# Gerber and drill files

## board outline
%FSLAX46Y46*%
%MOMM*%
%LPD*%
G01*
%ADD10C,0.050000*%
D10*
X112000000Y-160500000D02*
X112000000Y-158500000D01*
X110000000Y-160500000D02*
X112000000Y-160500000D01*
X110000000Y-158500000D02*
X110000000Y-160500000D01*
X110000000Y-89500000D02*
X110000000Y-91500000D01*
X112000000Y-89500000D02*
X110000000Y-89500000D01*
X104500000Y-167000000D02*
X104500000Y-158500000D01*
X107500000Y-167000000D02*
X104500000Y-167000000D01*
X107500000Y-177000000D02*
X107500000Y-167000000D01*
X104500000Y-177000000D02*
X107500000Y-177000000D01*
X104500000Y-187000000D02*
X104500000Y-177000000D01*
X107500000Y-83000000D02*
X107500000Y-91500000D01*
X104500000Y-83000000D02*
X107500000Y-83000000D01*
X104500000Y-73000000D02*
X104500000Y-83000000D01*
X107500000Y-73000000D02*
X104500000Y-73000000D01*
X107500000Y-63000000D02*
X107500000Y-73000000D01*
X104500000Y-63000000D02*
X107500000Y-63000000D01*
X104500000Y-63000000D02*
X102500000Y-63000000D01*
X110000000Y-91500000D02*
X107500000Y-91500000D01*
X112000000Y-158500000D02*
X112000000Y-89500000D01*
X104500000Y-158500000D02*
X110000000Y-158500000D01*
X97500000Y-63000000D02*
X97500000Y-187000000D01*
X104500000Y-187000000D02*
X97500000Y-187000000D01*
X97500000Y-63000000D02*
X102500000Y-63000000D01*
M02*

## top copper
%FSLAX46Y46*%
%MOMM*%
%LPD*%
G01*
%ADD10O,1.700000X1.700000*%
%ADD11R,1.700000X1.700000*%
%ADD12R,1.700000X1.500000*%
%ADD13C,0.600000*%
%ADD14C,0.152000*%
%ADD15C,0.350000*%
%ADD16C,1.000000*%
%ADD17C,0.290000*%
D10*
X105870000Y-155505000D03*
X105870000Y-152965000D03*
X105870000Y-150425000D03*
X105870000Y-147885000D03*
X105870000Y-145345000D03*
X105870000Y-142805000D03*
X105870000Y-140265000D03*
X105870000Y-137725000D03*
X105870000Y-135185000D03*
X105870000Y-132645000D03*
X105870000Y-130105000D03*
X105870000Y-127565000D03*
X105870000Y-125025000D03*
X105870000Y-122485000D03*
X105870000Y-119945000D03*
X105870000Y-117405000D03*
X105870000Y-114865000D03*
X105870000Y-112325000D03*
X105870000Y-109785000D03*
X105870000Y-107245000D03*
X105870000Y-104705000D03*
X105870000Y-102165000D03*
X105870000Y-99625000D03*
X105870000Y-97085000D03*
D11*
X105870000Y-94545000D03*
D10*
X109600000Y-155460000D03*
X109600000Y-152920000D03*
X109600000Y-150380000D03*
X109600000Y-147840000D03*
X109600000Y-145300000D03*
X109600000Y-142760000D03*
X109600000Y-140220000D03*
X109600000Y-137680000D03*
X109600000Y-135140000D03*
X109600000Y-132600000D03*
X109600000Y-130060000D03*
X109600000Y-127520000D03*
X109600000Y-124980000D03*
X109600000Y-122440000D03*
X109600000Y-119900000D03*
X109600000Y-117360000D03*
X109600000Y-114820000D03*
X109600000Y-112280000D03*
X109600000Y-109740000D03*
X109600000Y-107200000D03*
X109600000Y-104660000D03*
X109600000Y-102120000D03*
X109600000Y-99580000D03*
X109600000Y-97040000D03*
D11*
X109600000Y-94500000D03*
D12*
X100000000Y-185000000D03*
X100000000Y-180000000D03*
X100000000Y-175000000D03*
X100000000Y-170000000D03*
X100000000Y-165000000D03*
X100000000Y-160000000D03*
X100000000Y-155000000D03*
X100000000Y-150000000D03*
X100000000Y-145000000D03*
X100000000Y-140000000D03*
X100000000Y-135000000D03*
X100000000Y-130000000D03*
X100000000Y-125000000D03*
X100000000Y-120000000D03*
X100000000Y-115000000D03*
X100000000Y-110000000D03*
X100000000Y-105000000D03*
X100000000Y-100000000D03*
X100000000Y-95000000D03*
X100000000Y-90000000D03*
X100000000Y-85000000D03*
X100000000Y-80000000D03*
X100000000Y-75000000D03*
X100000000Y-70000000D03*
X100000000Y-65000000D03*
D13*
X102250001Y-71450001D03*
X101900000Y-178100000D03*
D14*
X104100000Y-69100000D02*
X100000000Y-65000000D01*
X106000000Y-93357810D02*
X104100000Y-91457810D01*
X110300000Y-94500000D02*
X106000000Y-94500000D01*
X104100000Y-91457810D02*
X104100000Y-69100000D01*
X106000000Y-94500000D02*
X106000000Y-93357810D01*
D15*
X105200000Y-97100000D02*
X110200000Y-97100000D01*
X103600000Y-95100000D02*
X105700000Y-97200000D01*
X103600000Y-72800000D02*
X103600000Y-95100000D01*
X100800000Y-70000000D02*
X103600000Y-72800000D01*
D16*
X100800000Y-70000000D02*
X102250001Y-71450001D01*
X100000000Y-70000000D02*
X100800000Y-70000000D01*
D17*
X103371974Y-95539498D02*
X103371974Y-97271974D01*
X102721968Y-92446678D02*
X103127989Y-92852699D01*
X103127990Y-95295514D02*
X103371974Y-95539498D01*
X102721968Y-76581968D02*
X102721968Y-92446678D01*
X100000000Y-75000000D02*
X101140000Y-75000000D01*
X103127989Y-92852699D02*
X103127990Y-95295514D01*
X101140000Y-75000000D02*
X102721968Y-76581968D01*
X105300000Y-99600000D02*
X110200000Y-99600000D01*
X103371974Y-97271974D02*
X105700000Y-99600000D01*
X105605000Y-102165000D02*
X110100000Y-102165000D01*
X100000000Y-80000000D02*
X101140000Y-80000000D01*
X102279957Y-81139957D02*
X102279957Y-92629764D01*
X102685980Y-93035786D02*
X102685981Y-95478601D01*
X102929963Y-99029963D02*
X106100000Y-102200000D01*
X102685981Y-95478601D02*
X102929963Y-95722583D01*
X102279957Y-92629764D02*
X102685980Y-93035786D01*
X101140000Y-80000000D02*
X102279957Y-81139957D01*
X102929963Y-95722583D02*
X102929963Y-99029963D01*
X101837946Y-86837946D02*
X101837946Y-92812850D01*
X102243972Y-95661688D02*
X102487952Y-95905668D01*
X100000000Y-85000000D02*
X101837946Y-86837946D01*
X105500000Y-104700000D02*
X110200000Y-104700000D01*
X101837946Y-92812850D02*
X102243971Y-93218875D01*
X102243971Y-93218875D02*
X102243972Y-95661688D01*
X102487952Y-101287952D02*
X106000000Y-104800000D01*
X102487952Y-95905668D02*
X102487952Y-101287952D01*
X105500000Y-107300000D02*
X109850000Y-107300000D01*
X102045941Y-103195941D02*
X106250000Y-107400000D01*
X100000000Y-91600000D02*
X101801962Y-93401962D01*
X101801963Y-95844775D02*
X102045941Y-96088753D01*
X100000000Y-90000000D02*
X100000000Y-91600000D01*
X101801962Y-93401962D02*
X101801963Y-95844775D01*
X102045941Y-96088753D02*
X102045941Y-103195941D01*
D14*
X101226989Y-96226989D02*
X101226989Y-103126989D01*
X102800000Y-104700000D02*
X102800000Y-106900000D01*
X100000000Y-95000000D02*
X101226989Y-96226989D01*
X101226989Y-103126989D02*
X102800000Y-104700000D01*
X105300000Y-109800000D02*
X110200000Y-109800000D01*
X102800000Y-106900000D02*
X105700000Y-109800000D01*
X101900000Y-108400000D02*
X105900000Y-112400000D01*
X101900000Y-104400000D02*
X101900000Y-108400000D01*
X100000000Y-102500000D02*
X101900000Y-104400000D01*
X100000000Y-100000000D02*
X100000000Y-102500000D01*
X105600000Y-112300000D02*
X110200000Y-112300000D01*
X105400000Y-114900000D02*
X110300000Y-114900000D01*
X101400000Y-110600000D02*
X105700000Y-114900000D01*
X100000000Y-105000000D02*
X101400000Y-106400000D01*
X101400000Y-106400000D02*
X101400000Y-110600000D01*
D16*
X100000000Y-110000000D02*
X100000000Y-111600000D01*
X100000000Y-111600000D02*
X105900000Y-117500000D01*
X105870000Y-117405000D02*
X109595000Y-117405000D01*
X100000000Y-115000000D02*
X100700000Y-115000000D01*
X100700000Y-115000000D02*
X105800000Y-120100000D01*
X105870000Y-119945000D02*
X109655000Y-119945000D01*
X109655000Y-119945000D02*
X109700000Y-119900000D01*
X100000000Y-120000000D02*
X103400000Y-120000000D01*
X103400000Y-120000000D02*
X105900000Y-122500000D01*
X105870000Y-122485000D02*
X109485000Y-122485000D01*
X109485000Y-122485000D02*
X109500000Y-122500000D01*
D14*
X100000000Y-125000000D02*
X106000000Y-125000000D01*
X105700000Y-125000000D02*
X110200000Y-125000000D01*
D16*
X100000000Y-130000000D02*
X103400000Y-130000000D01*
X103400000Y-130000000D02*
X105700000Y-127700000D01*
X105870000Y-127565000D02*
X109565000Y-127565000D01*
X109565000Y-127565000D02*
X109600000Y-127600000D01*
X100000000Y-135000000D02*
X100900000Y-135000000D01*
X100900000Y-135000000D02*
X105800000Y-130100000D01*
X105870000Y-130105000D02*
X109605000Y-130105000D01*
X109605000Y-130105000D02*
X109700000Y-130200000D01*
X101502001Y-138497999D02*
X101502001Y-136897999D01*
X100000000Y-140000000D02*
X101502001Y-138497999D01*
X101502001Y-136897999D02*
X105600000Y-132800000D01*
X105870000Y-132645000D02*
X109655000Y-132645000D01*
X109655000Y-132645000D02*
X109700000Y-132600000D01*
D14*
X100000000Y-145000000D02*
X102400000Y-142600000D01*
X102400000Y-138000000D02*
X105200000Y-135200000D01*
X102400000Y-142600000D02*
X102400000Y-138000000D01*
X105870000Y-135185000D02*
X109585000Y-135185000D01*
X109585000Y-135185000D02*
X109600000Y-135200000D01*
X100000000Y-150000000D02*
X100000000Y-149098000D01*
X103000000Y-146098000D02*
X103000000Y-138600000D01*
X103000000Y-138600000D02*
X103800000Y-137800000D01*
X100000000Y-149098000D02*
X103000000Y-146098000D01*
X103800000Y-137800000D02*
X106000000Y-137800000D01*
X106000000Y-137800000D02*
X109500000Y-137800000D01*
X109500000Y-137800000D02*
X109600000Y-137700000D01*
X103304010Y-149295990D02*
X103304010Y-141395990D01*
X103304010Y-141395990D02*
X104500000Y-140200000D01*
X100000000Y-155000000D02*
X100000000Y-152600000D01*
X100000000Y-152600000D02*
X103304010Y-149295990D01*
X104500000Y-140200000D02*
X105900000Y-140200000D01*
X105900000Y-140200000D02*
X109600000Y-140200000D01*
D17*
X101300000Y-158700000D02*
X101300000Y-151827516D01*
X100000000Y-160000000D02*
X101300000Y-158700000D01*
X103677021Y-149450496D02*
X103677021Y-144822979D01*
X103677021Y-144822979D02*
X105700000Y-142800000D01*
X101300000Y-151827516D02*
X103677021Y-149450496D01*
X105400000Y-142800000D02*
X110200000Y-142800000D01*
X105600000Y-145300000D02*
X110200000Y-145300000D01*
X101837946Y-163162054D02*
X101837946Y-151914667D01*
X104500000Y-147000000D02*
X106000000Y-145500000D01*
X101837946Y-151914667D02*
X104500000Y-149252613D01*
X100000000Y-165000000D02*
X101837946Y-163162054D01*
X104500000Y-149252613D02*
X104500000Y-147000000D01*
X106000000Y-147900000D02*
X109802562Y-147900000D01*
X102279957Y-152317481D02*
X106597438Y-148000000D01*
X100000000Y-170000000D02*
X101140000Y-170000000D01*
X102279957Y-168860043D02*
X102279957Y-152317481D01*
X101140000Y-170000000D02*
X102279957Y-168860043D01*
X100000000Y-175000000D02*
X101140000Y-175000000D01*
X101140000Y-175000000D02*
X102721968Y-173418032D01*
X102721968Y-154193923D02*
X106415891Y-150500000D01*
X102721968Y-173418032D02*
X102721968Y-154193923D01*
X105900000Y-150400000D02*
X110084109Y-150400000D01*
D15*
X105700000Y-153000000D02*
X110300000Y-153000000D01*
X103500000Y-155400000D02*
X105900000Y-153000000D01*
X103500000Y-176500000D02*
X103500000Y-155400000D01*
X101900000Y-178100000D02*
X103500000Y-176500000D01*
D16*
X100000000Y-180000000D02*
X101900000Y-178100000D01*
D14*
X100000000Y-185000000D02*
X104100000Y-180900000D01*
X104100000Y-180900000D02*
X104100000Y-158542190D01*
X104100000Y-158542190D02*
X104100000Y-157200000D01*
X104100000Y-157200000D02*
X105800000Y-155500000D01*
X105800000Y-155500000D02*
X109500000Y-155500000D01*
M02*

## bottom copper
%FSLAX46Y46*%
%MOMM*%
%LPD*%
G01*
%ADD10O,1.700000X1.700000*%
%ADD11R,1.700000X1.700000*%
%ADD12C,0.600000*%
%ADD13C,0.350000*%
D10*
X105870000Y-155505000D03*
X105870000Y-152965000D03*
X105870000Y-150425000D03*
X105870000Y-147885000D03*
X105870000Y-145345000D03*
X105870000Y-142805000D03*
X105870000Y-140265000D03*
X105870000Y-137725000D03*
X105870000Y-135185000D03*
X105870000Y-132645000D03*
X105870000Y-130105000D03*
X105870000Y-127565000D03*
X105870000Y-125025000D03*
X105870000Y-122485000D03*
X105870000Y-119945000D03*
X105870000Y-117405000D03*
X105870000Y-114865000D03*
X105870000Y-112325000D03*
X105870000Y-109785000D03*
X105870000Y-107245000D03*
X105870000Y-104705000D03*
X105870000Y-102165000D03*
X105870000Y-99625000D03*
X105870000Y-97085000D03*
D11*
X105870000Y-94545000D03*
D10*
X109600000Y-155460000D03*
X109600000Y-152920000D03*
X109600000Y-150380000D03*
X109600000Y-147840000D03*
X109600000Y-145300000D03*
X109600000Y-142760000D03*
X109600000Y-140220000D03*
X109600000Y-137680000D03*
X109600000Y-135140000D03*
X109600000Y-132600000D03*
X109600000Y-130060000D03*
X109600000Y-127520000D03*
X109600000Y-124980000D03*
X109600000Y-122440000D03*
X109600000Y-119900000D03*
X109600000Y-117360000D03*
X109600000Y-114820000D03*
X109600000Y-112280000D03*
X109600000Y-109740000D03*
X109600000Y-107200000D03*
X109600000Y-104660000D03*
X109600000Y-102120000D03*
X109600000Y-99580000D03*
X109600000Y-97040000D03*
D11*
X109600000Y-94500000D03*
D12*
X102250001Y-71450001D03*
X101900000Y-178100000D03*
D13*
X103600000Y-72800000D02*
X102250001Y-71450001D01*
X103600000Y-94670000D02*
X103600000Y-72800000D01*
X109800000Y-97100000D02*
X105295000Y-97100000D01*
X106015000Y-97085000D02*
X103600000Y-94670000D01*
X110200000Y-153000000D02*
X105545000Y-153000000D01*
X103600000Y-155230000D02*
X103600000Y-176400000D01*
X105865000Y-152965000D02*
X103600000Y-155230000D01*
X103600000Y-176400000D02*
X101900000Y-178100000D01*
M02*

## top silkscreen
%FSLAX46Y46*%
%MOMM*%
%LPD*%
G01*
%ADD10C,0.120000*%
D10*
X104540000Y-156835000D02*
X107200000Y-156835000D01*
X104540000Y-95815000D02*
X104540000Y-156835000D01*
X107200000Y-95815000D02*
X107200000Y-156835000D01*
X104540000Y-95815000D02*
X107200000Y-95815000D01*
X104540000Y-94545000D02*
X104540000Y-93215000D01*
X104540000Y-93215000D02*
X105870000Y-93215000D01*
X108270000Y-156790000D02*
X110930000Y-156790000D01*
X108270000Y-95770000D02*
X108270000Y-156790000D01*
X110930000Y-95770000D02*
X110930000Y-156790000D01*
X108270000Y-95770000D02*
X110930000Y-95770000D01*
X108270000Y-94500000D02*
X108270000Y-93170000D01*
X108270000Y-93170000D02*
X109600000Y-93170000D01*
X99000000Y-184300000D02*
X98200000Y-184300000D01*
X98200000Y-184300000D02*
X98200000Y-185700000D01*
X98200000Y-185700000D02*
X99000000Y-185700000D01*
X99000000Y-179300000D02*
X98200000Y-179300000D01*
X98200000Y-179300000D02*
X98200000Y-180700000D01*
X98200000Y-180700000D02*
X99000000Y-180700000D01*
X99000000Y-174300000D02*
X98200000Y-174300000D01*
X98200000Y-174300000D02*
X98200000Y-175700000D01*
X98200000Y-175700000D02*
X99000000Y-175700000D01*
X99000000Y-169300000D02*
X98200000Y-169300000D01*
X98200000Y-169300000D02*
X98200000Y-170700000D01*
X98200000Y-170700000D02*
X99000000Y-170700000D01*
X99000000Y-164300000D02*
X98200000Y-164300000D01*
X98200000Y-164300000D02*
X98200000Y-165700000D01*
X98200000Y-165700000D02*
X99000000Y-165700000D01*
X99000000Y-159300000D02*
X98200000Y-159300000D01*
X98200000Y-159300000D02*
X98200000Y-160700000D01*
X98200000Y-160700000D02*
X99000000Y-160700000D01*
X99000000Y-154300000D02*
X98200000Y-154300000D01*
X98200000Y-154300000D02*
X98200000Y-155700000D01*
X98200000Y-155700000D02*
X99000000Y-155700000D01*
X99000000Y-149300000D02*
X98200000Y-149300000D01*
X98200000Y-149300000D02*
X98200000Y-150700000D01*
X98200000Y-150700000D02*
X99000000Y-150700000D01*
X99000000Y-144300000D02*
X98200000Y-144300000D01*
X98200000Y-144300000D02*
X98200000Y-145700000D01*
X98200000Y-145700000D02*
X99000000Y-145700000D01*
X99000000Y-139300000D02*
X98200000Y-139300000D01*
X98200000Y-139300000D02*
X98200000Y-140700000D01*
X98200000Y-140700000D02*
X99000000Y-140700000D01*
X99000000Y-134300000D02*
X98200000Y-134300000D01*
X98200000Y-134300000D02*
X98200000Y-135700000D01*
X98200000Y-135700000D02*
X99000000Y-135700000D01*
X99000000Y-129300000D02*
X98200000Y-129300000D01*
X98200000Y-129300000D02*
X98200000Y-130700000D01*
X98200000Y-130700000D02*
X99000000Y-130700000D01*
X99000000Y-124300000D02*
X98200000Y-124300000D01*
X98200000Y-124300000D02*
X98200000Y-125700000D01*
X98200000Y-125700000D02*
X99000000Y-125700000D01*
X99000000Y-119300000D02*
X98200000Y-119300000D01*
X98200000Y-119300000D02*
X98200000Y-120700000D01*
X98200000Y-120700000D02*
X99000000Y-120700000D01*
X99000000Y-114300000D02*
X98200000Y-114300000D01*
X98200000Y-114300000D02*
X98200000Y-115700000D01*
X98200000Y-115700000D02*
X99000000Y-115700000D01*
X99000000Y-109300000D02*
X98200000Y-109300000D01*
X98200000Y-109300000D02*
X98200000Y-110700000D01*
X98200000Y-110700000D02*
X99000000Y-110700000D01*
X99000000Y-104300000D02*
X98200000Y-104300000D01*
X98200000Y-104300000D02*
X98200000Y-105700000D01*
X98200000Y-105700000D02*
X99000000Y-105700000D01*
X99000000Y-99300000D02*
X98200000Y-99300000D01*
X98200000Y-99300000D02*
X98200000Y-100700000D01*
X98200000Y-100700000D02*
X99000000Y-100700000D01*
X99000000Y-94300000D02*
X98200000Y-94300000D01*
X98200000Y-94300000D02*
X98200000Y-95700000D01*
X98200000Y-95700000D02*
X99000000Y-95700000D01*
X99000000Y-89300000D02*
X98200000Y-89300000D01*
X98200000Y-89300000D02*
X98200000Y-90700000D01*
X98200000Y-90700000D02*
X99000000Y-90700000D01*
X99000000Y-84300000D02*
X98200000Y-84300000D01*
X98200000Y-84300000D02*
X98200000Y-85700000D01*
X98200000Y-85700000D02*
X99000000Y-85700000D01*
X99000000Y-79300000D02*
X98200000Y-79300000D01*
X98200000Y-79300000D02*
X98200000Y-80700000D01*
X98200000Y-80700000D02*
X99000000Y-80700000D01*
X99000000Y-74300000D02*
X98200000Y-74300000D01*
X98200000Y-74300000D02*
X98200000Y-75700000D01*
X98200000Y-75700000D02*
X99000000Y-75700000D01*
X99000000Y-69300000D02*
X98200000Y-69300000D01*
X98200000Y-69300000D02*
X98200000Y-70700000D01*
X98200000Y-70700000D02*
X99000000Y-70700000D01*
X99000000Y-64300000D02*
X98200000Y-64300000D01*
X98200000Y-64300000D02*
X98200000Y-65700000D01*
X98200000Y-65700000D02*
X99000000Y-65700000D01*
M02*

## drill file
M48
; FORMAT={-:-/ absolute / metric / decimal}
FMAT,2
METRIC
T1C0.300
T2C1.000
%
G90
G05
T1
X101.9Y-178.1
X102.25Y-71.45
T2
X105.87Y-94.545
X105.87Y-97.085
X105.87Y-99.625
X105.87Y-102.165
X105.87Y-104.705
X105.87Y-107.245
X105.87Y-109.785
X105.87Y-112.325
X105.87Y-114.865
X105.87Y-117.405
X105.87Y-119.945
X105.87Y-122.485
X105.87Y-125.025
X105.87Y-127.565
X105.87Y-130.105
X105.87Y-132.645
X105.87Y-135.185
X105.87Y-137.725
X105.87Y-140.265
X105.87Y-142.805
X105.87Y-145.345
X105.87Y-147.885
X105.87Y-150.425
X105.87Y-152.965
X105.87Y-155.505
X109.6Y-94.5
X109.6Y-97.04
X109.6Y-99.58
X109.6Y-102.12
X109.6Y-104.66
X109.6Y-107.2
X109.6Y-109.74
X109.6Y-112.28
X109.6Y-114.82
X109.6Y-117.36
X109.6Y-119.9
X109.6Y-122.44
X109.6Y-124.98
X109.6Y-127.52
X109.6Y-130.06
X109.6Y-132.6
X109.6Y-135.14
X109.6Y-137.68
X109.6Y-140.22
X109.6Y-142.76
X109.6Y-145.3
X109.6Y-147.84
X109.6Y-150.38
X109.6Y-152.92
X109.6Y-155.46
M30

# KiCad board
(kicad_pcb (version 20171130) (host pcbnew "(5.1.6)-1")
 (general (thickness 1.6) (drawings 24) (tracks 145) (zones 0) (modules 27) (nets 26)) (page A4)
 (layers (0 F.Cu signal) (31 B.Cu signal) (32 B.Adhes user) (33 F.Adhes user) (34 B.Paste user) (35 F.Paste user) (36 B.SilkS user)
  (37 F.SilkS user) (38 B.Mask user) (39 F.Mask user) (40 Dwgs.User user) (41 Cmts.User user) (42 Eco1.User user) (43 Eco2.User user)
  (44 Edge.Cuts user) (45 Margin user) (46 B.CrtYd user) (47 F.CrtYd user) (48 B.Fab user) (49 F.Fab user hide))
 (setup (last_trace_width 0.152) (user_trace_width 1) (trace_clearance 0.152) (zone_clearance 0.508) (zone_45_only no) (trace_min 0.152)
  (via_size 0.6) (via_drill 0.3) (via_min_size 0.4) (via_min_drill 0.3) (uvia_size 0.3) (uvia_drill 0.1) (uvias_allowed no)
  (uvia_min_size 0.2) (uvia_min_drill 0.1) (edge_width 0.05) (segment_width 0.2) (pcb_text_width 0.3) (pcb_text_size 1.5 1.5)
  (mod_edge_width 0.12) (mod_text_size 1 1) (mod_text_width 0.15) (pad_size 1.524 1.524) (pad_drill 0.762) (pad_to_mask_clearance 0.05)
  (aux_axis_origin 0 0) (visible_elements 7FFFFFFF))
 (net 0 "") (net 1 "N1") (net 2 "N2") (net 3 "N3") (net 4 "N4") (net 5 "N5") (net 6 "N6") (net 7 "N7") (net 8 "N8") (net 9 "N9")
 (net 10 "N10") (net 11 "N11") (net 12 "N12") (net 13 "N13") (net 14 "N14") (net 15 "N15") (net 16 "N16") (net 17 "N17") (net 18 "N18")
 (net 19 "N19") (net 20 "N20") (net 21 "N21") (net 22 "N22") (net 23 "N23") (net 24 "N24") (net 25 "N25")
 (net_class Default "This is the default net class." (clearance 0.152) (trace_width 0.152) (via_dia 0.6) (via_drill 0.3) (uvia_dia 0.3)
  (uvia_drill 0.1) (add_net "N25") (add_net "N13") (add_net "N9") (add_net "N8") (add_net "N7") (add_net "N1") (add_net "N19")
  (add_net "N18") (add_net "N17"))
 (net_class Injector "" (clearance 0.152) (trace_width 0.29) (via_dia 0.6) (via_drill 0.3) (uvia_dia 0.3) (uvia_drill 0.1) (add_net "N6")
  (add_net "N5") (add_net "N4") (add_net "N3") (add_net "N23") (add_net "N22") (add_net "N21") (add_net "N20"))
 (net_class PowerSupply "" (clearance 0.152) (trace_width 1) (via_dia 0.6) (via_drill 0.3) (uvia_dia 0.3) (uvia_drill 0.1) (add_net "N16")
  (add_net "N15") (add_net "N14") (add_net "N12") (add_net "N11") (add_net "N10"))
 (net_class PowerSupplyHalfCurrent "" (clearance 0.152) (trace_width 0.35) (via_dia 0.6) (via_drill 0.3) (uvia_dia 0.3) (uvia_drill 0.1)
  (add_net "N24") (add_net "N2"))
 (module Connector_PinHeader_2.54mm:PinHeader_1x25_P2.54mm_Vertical (layer F.Cu) (at 105.87 94.545)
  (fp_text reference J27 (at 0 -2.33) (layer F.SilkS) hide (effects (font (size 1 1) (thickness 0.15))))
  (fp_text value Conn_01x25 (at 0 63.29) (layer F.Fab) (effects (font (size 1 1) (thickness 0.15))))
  (fp_line (start -1.33 62.29) (end 1.33 62.29) (layer F.SilkS) (width 0.12))
  (fp_line (start -1.33 1.27) (end -1.33 62.29) (layer F.SilkS) (width 0.12))
  (fp_line (start 1.33 1.27) (end 1.33 62.29) (layer F.SilkS) (width 0.12))
  (fp_line (start -1.33 1.27) (end 1.33 1.27) (layer F.SilkS) (width 0.12))
  (fp_line (start -1.33 0) (end -1.33 -1.33) (layer F.SilkS) (width 0.12))
  (fp_line (start -1.33 -1.33) (end 0 -1.33) (layer F.SilkS) (width 0.12))
  (pad 25 thru_hole oval (at 0 60.96) (size 1.7 1.7) (drill 1) (layers *.Cu *.Mask) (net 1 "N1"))
  (pad 24 thru_hole oval (at 0 58.42) (size 1.7 1.7) (drill 1) (layers *.Cu *.Mask) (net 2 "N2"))
  (pad 23 thru_hole oval (at 0 55.88) (size 1.7 1.7) (drill 1) (layers *.Cu *.Mask) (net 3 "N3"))
  (pad 22 thru_hole oval (at 0 53.34) (size 1.7 1.7) (drill 1) (layers *.Cu *.Mask) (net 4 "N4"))
  (pad 21 thru_hole oval (at 0 50.8) (size 1.7 1.7) (drill 1) (layers *.Cu *.Mask) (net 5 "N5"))
  (pad 20 thru_hole oval (at 0 48.26) (size 1.7 1.7) (drill 1) (layers *.Cu *.Mask) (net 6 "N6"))
  (pad 19 thru_hole oval (at 0 45.72) (size 1.7 1.7) (drill 1) (layers *.Cu *.Mask) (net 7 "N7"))
  (pad 18 thru_hole oval (at 0 43.18) (size 1.7 1.7) (drill 1) (layers *.Cu *.Mask) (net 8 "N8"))
  (pad 17 thru_hole oval (at 0 40.64) (size 1.7 1.7) (drill 1) (layers *.Cu *.Mask) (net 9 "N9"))
  (pad 16 thru_hole oval (at 0 38.1) (size 1.7 1.7) (drill 1) (layers *.Cu *.Mask) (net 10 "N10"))
  (pad 15 thru_hole oval (at 0 35.56) (size 1.7 1.7) (drill 1) (layers *.Cu *.Mask) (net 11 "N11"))
  (pad 14 thru_hole oval (at 0 33.02) (size 1.7 1.7) (drill 1) (layers *.Cu *.Mask) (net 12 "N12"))
  (pad 13 thru_hole oval (at 0 30.48) (size 1.7 1.7) (drill 1) (layers *.Cu *.Mask) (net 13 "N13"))
  (pad 12 thru_hole oval (at 0 27.94) (size 1.7 1.7) (drill 1) (layers *.Cu *.Mask) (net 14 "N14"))
  (pad 11 thru_hole oval (at 0 25.4) (size 1.7 1.7) (drill 1) (layers *.Cu *.Mask) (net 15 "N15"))
  (pad 10 thru_hole oval (at 0 22.86) (size 1.7 1.7) (drill 1) (layers *.Cu *.Mask) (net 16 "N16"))
  (pad 9 thru_hole oval (at 0 20.32) (size 1.7 1.7) (drill 1) (layers *.Cu *.Mask) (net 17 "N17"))
  (pad 8 thru_hole oval (at 0 17.78) (size 1.7 1.7) (drill 1) (layers *.Cu *.Mask) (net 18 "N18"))
  (pad 7 thru_hole oval (at 0 15.24) (size 1.7 1.7) (drill 1) (layers *.Cu *.Mask) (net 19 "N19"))
  (pad 6 thru_hole oval (at 0 12.7) (size 1.7 1.7) (drill 1) (layers *.Cu *.Mask) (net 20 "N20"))
  (pad 5 thru_hole oval (at 0 10.16) (size 1.7 1.7) (drill 1) (layers *.Cu *.Mask) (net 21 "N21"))
  (pad 4 thru_hole oval (at 0 7.62) (size 1.7 1.7) (drill 1) (layers *.Cu *.Mask) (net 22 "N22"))
  (pad 3 thru_hole oval (at 0 5.08) (size 1.7 1.7) (drill 1) (layers *.Cu *.Mask) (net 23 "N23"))
  (pad 2 thru_hole oval (at 0 2.54) (size 1.7 1.7) (drill 1) (layers *.Cu *.Mask) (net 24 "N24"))
  (pad 1 thru_hole rect (at 0 0) (size 1.7 1.7) (drill 1) (layers *.Cu *.Mask) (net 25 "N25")))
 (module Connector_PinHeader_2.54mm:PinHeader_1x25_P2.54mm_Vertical (layer F.Cu) (at 109.6 94.5)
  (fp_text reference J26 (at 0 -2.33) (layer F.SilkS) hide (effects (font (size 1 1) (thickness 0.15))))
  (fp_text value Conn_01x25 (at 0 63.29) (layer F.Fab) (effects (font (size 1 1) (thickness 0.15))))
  (fp_line (start -1.33 62.29) (end 1.33 62.29) (layer F.SilkS) (width 0.12))
  (fp_line (start -1.33 1.27) (end -1.33 62.29) (layer F.SilkS) (width 0.12))
  (fp_line (start 1.33 1.27) (end 1.33 62.29) (layer F.SilkS) (width 0.12))
  (fp_line (start -1.33 1.27) (end 1.33 1.27) (layer F.SilkS) (width 0.12))
  (fp_line (start -1.33 0) (end -1.33 -1.33) (layer F.SilkS) (width 0.12))
  (fp_line (start -1.33 -1.33) (end 0 -1.33) (layer F.SilkS) (width 0.12))
  (pad 25 thru_hole oval (at 0 60.96) (size 1.7 1.7) (drill 1) (layers *.Cu *.Mask) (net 1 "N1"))
  (pad 24 thru_hole oval (at 0 58.42) (size 1.7 1.7) (drill 1) (layers *.Cu *.Mask) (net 2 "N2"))
  (pad 23 thru_hole oval (at 0 55.88) (size 1.7 1.7) (drill 1) (layers *.Cu *.Mask) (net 3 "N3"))
  (pad 22 thru_hole oval (at 0 53.34) (size 1.7 1.7) (drill 1) (layers *.Cu *.Mask) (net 4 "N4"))
  (pad 21 thru_hole oval (at 0 50.8) (size 1.7 1.7) (drill 1) (layers *.Cu *.Mask) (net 5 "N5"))
  (pad 20 thru_hole oval (at 0 48.26) (size 1.7 1.7) (drill 1) (layers *.Cu *.Mask) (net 6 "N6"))
  (pad 19 thru_hole oval (at 0 45.72) (size 1.7 1.7) (drill 1) (layers *.Cu *.Mask) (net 7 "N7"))
  (pad 18 thru_hole oval (at 0 43.18) (size 1.7 1.7) (drill 1) (layers *.Cu *.Mask) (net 8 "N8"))
  (pad 17 thru_hole oval (at 0 40.64) (size 1.7 1.7) (drill 1) (layers *.Cu *.Mask) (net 9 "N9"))
  (pad 16 thru_hole oval (at 0 38.1) (size 1.7 1.7) (drill 1) (layers *.Cu *.Mask) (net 10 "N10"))
  (pad 15 thru_hole oval (at 0 35.56) (size 1.7 1.7) (drill 1) (layers *.Cu *.Mask) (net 11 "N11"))
  (pad 14 thru_hole oval (at 0 33.02) (size 1.7 1.7) (drill 1) (layers *.Cu *.Mask) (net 12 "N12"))
  (pad 13 thru_hole oval (at 0 30.48) (size 1.7 1.7) (drill 1) (layers *.Cu *.Mask) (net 13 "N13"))
  (pad 12 thru_hole oval (at 0 27.94) (size 1.7 1.7) (drill 1) (layers *.Cu *.Mask) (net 14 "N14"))
  (pad 11 thru_hole oval (at 0 25.4) (size 1.7 1.7) (drill 1) (layers *.Cu *.Mask) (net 15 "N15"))
  (pad 10 thru_hole oval (at 0 22.86) (size 1.7 1.7) (drill 1) (layers *.Cu *.Mask) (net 16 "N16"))
  (pad 9 thru_hole oval (at 0 20.32) (size 1.7 1.7) (drill 1) (layers *.Cu *.Mask) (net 17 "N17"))
  (pad 8 thru_hole oval (at 0 17.78) (size 1.7 1.7) (drill 1) (layers *.Cu *.Mask) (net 18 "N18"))
  (pad 7 thru_hole oval (at 0 15.24) (size 1.7 1.7) (drill 1) (layers *.Cu *.Mask) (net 19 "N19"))
  (pad 6 thru_hole oval (at 0 12.7) (size 1.7 1.7) (drill 1) (layers *.Cu *.Mask) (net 20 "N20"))
  (pad 5 thru_hole oval (at 0 10.16) (size 1.7 1.7) (drill 1) (layers *.Cu *.Mask) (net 21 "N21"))
  (pad 4 thru_hole oval (at 0 7.62) (size 1.7 1.7) (drill 1) (layers *.Cu *.Mask) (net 22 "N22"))
  (pad 3 thru_hole oval (at 0 5.08) (size 1.7 1.7) (drill 1) (layers *.Cu *.Mask) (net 23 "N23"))
  (pad 2 thru_hole oval (at 0 2.54) (size 1.7 1.7) (drill 1) (layers *.Cu *.Mask) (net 24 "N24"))
  (pad 1 thru_hole rect (at 0 0) (size 1.7 1.7) (drill 1) (layers *.Cu *.Mask) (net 25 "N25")))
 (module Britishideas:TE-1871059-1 (layer F.Cu) (at 100 185)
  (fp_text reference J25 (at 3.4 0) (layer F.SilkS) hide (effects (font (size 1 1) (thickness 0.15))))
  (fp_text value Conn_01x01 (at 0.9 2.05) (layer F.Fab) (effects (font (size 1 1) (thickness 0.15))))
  (fp_line (start -1 -0.7) (end -1.8 -0.7) (layer F.SilkS) (width 0.12))
  (fp_line (start -1.8 -0.7) (end -1.8 0.7) (layer F.SilkS) (width 0.12))
  (fp_line (start -1.8 0.7) (end -1 0.7) (layer F.SilkS) (width 0.12))
  (pad 1 smd rect (at 0 0) (size 1.7 1.5) (layers F.Cu F.Paste F.Mask) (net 1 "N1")))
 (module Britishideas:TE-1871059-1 (layer F.Cu) (at 100 180)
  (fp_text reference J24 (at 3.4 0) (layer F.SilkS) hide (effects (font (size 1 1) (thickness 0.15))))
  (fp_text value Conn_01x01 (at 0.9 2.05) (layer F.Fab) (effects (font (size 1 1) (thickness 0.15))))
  (fp_line (start -1 -0.7) (end -1.8 -0.7) (layer F.SilkS) (width 0.12))
  (fp_line (start -1.8 -0.7) (end -1.8 0.7) (layer F.SilkS) (width 0.12))
  (fp_line (start -1.8 0.7) (end -1 0.7) (layer F.SilkS) (width 0.12))
  (pad 1 smd rect (at 0 0) (size 1.7 1.5) (layers F.Cu F.Paste F.Mask) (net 2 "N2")))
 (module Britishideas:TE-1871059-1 (layer F.Cu) (at 100 175)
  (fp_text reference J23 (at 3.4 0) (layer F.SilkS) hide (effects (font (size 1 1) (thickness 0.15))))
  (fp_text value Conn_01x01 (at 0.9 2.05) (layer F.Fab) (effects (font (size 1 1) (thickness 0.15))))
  (fp_line (start -1 -0.7) (end -1.8 -0.7) (layer F.SilkS) (width 0.12))
  (fp_line (start -1.8 -0.7) (end -1.8 0.7) (layer F.SilkS) (width 0.12))
  (fp_line (start -1.8 0.7) (end -1 0.7) (layer F.SilkS) (width 0.12))
  (pad 1 smd rect (at 0 0) (size 1.7 1.5) (layers F.Cu F.Paste F.Mask) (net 3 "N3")))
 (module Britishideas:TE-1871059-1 (layer F.Cu) (at 100 170)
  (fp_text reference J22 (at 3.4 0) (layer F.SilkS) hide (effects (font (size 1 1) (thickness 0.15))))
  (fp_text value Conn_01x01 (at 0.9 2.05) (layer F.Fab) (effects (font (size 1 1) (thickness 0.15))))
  (fp_line (start -1 -0.7) (end -1.8 -0.7) (layer F.SilkS) (width 0.12))
  (fp_line (start -1.8 -0.7) (end -1.8 0.7) (layer F.SilkS) (width 0.12))
  (fp_line (start -1.8 0.7) (end -1 0.7) (layer F.SilkS) (width 0.12))
  (pad 1 smd rect (at 0 0) (size 1.7 1.5) (layers F.Cu F.Paste F.Mask) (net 4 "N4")))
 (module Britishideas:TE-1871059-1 (layer F.Cu) (at 100 165)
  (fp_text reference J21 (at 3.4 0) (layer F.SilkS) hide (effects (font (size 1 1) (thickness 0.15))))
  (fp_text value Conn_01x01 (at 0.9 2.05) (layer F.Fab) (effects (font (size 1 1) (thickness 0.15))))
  (fp_line (start -1 -0.7) (end -1.8 -0.7) (layer F.SilkS) (width 0.12))
  (fp_line (start -1.8 -0.7) (end -1.8 0.7) (layer F.SilkS) (width 0.12))
  (fp_line (start -1.8 0.7) (end -1 0.7) (layer F.SilkS) (width 0.12))
  (pad 1 smd rect (at 0 0) (size 1.7 1.5) (layers F.Cu F.Paste F.Mask) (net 5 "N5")))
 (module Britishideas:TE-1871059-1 (layer F.Cu) (at 100 160)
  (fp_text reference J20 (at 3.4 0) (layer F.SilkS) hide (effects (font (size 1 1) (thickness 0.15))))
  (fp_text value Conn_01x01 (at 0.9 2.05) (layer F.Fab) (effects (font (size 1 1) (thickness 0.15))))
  (fp_line (start -1 -0.7) (end -1.8 -0.7) (layer F.SilkS) (width 0.12))
  (fp_line (start -1.8 -0.7) (end -1.8 0.7) (layer F.SilkS) (width 0.12))
  (fp_line (start -1.8 0.7) (end -1 0.7) (layer F.SilkS) (width 0.12))
  (pad 1 smd rect (at 0 0) (size 1.7 1.5) (layers F.Cu F.Paste F.Mask) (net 6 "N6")))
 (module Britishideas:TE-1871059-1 (layer F.Cu) (at 100 155)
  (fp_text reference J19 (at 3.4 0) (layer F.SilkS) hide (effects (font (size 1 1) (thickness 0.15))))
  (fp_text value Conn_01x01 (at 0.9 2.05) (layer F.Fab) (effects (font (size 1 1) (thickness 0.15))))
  (fp_line (start -1 -0.7) (end -1.8 -0.7) (layer F.SilkS) (width 0.12))
  (fp_line (start -1.8 -0.7) (end -1.8 0.7) (layer F.SilkS) (width 0.12))
  (fp_line (start -1.8 0.7) (end -1 0.7) (layer F.SilkS) (width 0.12))
  (pad 1 smd rect (at 0 0) (size 1.7 1.5) (layers F.Cu F.Paste F.Mask) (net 7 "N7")))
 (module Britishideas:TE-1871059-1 (layer F.Cu) (at 100 150)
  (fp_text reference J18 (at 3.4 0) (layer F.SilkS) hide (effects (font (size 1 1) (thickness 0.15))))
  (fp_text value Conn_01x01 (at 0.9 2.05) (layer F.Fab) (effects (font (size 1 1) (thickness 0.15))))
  (fp_line (start -1 -0.7) (end -1.8 -0.7) (layer F.SilkS) (width 0.12))
  (fp_line (start -1.8 -0.7) (end -1.8 0.7) (layer F.SilkS) (width 0.12))
  (fp_line (start -1.8 0.7) (end -1 0.7) (layer F.SilkS) (width 0.12))
  (pad 1 smd rect (at 0 0) (size 1.7 1.5) (layers F.Cu F.Paste F.Mask) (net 8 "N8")))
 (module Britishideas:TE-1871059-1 (layer F.Cu) (at 100 145)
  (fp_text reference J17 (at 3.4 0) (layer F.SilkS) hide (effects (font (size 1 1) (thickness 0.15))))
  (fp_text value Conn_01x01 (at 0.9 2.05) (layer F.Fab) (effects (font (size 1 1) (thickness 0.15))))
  (fp_line (start -1 -0.7) (end -1.8 -0.7) (layer F.SilkS) (width 0.12))
  (fp_line (start -1.8 -0.7) (end -1.8 0.7) (layer F.SilkS) (width 0.12))
  (fp_line (start -1.8 0.7) (end -1 0.7) (layer F.SilkS) (width 0.12))
  (pad 1 smd rect (at 0 0) (size 1.7 1.5) (layers F.Cu F.Paste F.Mask) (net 9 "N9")))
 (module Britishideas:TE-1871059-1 (layer F.Cu) (at 100 140)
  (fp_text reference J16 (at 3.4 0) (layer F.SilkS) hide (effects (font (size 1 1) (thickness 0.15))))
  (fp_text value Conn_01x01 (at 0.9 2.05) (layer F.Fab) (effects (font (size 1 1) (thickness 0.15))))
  (fp_line (start -1 -0.7) (end -1.8 -0.7) (layer F.SilkS) (width 0.12))
  (fp_line (start -1.8 -0.7) (end -1.8 0.7) (layer F.SilkS) (width 0.12))
  (fp_line (start -1.8 0.7) (end -1 0.7) (layer F.SilkS) (width 0.12))
  (pad 1 smd rect (at 0 0) (size 1.7 1.5) (layers F.Cu F.Paste F.Mask) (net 10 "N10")))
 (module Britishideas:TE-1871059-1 (layer F.Cu) (at 100 135)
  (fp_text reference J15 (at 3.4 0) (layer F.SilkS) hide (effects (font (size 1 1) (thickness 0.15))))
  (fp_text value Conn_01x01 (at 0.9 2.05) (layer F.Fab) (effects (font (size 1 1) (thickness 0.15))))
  (fp_line (start -1 -0.7) (end -1.8 -0.7) (layer F.SilkS) (width 0.12))
  (fp_line (start -1.8 -0.7) (end -1.8 0.7) (layer F.SilkS) (width 0.12))
  (fp_line (start -1.8 0.7) (end -1 0.7) (layer F.SilkS) (width 0.12))
  (pad 1 smd rect (at 0 0) (size 1.7 1.5) (layers F.Cu F.Paste F.Mask) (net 11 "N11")))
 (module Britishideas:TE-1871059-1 (layer F.Cu) (at 100 130)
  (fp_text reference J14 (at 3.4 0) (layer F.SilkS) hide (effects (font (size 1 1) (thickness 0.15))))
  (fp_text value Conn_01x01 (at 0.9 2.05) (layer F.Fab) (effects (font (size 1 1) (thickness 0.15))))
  (fp_line (start -1 -0.7) (end -1.8 -0.7) (layer F.SilkS) (width 0.12))
  (fp_line (start -1.8 -0.7) (end -1.8 0.7) (layer F.SilkS) (width 0.12))
  (fp_line (start -1.8 0.7) (end -1 0.7) (layer F.SilkS) (width 0.12))
  (pad 1 smd rect (at 0 0) (size 1.7 1.5) (layers F.Cu F.Paste F.Mask) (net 12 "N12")))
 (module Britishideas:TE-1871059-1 (layer F.Cu) (at 100 125)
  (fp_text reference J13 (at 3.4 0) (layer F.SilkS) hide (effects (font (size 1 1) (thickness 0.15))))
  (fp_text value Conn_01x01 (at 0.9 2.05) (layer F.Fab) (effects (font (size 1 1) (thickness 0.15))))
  (fp_line (start -1 -0.7) (end -1.8 -0.7) (layer F.SilkS) (width 0.12))
  (fp_line (start -1.8 -0.7) (end -1.8 0.7) (layer F.SilkS) (width 0.12))
  (fp_line (start -1.8 0.7) (end -1 0.7) (layer F.SilkS) (width 0.12))
  (pad 1 smd rect (at 0 0) (size 1.7 1.5) (layers F.Cu F.Paste F.Mask) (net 13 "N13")))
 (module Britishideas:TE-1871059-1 (layer F.Cu) (at 100 120)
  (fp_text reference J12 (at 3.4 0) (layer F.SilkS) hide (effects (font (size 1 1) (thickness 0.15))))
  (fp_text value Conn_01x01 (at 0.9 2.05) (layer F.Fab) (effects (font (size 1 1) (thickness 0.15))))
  (fp_line (start -1 -0.7) (end -1.8 -0.7) (layer F.SilkS) (width 0.12))
  (fp_line (start -1.8 -0.7) (end -1.8 0.7) (layer F.SilkS) (width 0.12))
  (fp_line (start -1.8 0.7) (end -1 0.7) (layer F.SilkS) (width 0.12))
  (pad 1 smd rect (at 0 0) (size 1.7 1.5) (layers F.Cu F.Paste F.Mask) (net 14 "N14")))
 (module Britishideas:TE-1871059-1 (layer F.Cu) (at 100 115)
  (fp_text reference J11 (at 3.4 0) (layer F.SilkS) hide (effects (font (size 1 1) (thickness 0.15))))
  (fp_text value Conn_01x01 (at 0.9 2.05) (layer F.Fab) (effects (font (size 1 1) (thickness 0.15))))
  (fp_line (start -1 -0.7) (end -1.8 -0.7) (layer F.SilkS) (width 0.12))
  (fp_line (start -1.8 -0.7) (end -1.8 0.7) (layer F.SilkS) (width 0.12))
  (fp_line (start -1.8 0.7) (end -1 0.7) (layer F.SilkS) (width 0.12))
  (pad 1 smd rect (at 0 0) (size 1.7 1.5) (layers F.Cu F.Paste F.Mask) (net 15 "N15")))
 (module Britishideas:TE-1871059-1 (layer F.Cu) (at 100 110)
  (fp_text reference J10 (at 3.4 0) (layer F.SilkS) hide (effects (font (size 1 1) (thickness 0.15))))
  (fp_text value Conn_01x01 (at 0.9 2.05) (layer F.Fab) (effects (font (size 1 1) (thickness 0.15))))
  (fp_line (start -1 -0.7) (end -1.8 -0.7) (layer F.SilkS) (width 0.12))
  (fp_line (start -1.8 -0.7) (end -1.8 0.7) (layer F.SilkS) (width 0.12))
  (fp_line (start -1.8 0.7) (end -1 0.7) (layer F.SilkS) (width 0.12))
  (pad 1 smd rect (at 0 0) (size 1.7 1.5) (layers F.Cu F.Paste F.Mask) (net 16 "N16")))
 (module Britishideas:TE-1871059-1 (layer F.Cu) (at 100 105)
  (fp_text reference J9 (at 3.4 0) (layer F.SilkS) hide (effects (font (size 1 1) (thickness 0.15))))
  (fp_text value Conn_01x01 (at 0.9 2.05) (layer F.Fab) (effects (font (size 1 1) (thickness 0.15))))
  (fp_line (start -1 -0.7) (end -1.8 -0.7) (layer F.SilkS) (width 0.12))
  (fp_line (start -1.8 -0.7) (end -1.8 0.7) (layer F.SilkS) (width 0.12))
  (fp_line (start -1.8 0.7) (end -1 0.7) (layer F.SilkS) (width 0.12))
  (pad 1 smd rect (at 0 0) (size 1.7 1.5) (layers F.Cu F.Paste F.Mask) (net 17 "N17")))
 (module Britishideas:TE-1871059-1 (layer F.Cu) (at 100 100)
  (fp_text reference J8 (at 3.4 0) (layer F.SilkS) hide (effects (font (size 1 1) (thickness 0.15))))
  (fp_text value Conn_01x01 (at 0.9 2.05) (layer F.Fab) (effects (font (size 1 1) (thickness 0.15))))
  (fp_line (start -1 -0.7) (end -1.8 -0.7) (layer F.SilkS) (width 0.12))
  (fp_line (start -1.8 -0.7) (end -1.8 0.7) (layer F.SilkS) (width 0.12))
  (fp_line (start -1.8 0.7) (end -1 0.7) (layer F.SilkS) (width 0.12))
  (pad 1 smd rect (at 0 0) (size 1.7 1.5) (layers F.Cu F.Paste F.Mask) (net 18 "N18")))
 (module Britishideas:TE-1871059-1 (layer F.Cu) (at 100 95)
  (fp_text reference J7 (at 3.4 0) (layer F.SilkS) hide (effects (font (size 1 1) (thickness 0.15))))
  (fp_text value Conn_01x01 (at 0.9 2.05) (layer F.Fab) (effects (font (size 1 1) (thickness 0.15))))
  (fp_line (start -1 -0.7) (end -1.8 -0.7) (layer F.SilkS) (width 0.12))
  (fp_line (start -1.8 -0.7) (end -1.8 0.7) (layer F.SilkS) (width 0.12))
  (fp_line (start -1.8 0.7) (end -1 0.7) (layer F.SilkS) (width 0.12))
  (pad 1 smd rect (at 0 0) (size 1.7 1.5) (layers F.Cu F.Paste F.Mask) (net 19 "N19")))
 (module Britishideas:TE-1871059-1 (layer F.Cu) (at 100 90)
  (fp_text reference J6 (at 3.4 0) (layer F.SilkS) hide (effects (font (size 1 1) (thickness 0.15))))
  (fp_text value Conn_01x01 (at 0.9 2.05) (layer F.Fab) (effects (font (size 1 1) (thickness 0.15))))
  (fp_line (start -1 -0.7) (end -1.8 -0.7) (layer F.SilkS) (width 0.12))
  (fp_line (start -1.8 -0.7) (end -1.8 0.7) (layer F.SilkS) (width 0.12))
  (fp_line (start -1.8 0.7) (end -1 0.7) (layer F.SilkS) (width 0.12))
  (pad 1 smd rect (at 0 0) (size 1.7 1.5) (layers F.Cu F.Paste F.Mask) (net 20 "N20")))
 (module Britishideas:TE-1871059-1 (layer F.Cu) (at 100 85)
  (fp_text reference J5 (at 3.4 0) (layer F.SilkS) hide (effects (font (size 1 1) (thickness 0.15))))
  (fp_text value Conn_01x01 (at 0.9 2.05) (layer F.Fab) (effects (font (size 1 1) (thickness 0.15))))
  (fp_line (start -1 -0.7) (end -1.8 -0.7) (layer F.SilkS) (width 0.12))
  (fp_line (start -1.8 -0.7) (end -1.8 0.7) (layer F.SilkS) (width 0.12))
  (fp_line (start -1.8 0.7) (end -1 0.7) (layer F.SilkS) (width 0.12))
  (pad 1 smd rect (at 0 0) (size 1.7 1.5) (layers F.Cu F.Paste F.Mask) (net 21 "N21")))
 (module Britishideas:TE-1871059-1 (layer F.Cu) (at 100 80)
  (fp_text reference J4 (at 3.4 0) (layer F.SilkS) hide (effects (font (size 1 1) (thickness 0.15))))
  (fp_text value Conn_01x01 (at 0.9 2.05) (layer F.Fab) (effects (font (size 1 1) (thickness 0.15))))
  (fp_line (start -1 -0.7) (end -1.8 -0.7) (layer F.SilkS) (width 0.12))
  (fp_line (start -1.8 -0.7) (end -1.8 0.7) (layer F.SilkS) (width 0.12))
  (fp_line (start -1.8 0.7) (end -1 0.7) (layer F.SilkS) (width 0.12))
  (pad 1 smd rect (at 0 0) (size 1.7 1.5) (layers F.Cu F.Paste F.Mask) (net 22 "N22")))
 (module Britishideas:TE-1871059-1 (layer F.Cu) (at 100 75)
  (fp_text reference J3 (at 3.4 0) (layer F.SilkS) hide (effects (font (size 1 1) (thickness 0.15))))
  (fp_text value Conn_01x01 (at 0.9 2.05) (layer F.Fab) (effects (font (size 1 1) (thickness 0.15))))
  (fp_line (start -1 -0.7) (end -1.8 -0.7) (layer F.SilkS) (width 0.12))
  (fp_line (start -1.8 -0.7) (end -1.8 0.7) (layer F.SilkS) (width 0.12))
  (fp_line (start -1.8 0.7) (end -1 0.7) (layer F.SilkS) (width 0.12))
  (pad 1 smd rect (at 0 0) (size 1.7 1.5) (layers F.Cu F.Paste F.Mask) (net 23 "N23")))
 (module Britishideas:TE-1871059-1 (layer F.Cu) (at 100 70)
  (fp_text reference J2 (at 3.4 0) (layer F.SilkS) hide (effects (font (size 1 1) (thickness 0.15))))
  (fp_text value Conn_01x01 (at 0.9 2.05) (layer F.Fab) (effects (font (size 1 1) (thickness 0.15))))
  (fp_line (start -1 -0.7) (end -1.8 -0.7) (layer F.SilkS) (width 0.12))
  (fp_line (start -1.8 -0.7) (end -1.8 0.7) (layer F.SilkS) (width 0.12))
  (fp_line (start -1.8 0.7) (end -1 0.7) (layer F.SilkS) (width 0.12))
  (pad 1 smd rect (at 0 0) (size 1.7 1.5) (layers F.Cu F.Paste F.Mask) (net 24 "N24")))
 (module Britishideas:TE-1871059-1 (layer F.Cu) (at 100 65)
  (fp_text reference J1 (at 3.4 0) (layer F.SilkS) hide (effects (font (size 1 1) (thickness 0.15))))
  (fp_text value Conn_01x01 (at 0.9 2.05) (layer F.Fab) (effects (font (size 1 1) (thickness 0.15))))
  (fp_line (start -1 -0.7) (end -1.8 -0.7) (layer F.SilkS) (width 0.12))
  (fp_line (start -1.8 -0.7) (end -1.8 0.7) (layer F.SilkS) (width 0.12))
  (fp_line (start -1.8 0.7) (end -1 0.7) (layer F.SilkS) (width 0.12))
  (pad 1 smd rect (at 0 0) (size 1.7 1.5) (layers F.Cu F.Paste F.Mask) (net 25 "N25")))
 (gr_line (start 112 160.5) (end 112 158.5) (layer Edge.Cuts) (width 0.05))
 (gr_line (start 110 160.5) (end 112 160.5) (layer Edge.Cuts) (width 0.05))
 (gr_line (start 110 158.5) (end 110 160.5) (layer Edge.Cuts) (width 0.05))
 (gr_line (start 110 89.5) (end 110 91.5) (layer Edge.Cuts) (width 0.05))
 (gr_line (start 112 89.5) (end 110 89.5) (layer Edge.Cuts) (width 0.05))
 (gr_line (start 104.5 167) (end 104.5 158.5) (layer Edge.Cuts) (width 0.05))
 (gr_line (start 107.5 167) (end 104.5 167) (layer Edge.Cuts) (width 0.05))
 (gr_line (start 107.5 177) (end 107.5 167) (layer Edge.Cuts) (width 0.05))
 (gr_line (start 104.5 177) (end 107.5 177) (layer Edge.Cuts) (width 0.05))
 (gr_line (start 104.5 187) (end 104.5 177) (layer Edge.Cuts) (width 0.05))
 (gr_line (start 107.5 83) (end 107.5 91.5) (layer Edge.Cuts) (width 0.05))
 (gr_line (start 104.5 83) (end 107.5 83) (layer Edge.Cuts) (width 0.05))
 (gr_line (start 104.5 73) (end 104.5 83) (layer Edge.Cuts) (width 0.05))
 (gr_line (start 107.5 73) (end 104.5 73) (layer Edge.Cuts) (width 0.05))
 (gr_line (start 107.5 63) (end 107.5 73) (layer Edge.Cuts) (width 0.05))
 (gr_line (start 104.5 63) (end 107.5 63) (layer Edge.Cuts) (width 0.05))
 (gr_line (start 104.5 63) (end 102.5 63) (layer Edge.Cuts) (width 0.05))
 (gr_line (start 110 91.5) (end 107.5 91.5) (layer Edge.Cuts) (width 0.05))
 (gr_line (start 112 158.5) (end 112 89.5) (layer Edge.Cuts) (width 0.05))
 (gr_line (start 104.5 158.5) (end 110 158.5) (layer Edge.Cuts) (width 0.05))
 (gr_line (start 97.5 63) (end 97.5 187) (layer Edge.Cuts) (width 0.05))
 (gr_line (start 104.5 187) (end 97.5 187) (layer Edge.Cuts) (width 0.05))
 (gr_line (start 97.5 63) (end 102.5 63) (layer Edge.Cuts) (width 0.05))
 (segment (start 104.1 69.1) (end 100 65) (width 0.152) (layer F.Cu) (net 25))
 (segment (start 106 93.35781) (end 104.1 91.45781) (width 0.152) (layer F.Cu) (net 25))
 (segment (start 110.3 94.5) (end 106 94.5) (width 0.152) (layer F.Cu) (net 25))
 (segment (start 104.1 91.45781) (end 104.1 69.1) (width 0.152) (layer F.Cu) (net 25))
 (segment (start 106 94.5) (end 106 93.35781) (width 0.152) (layer F.Cu) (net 25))
 (via (at 102.250001 71.450001) (size 0.6) (drill 0.3) (layers F.Cu B.Cu) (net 24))
 (segment (start 103.6 72.8) (end 102.250001 71.450001) (width 0.35) (layer B.Cu) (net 24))
 (segment (start 103.6 94.67) (end 103.6 72.8) (width 0.35) (layer B.Cu) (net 24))
 (segment (start 109.8 97.1) (end 105.295 97.1) (width 0.35) (layer B.Cu) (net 24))
 (segment (start 106.015 97.085) (end 103.6 94.67) (width 0.35) (layer B.Cu) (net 24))
 (segment (start 105.2 97.1) (end 110.2 97.1) (width 0.35) (layer F.Cu) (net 24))
 (segment (start 103.6 95.1) (end 105.7 97.2) (width 0.35) (layer F.Cu) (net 24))
 (segment (start 103.6 72.8) (end 103.6 95.1) (width 0.35) (layer F.Cu) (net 24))
 (segment (start 100.8 70) (end 103.6 72.8) (width 0.35) (layer F.Cu) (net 24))
 (segment (start 100.8 70) (end 102.250001 71.450001) (width 1) (layer F.Cu) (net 24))
 (segment (start 100 70) (end 100.8 70) (width 1) (layer F.Cu) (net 24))
 (segment (start 103.371974 95.539498) (end 103.371974 97.271974) (width 0.29) (layer F.Cu) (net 23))
 (segment (start 102.721968 92.446678) (end 103.127989 92.852699) (width 0.29) (layer F.Cu) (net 23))
 (segment (start 103.12799 95.295514) (end 103.371974 95.539498) (width 0.29) (layer F.Cu) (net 23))
 (segment (start 102.721968 76.581968) (end 102.721968 92.446678) (width 0.29) (layer F.Cu) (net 23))
 (segment (start 100 75) (end 101.14 75) (width 0.29) (layer F.Cu) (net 23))
 (segment (start 103.127989 92.852699) (end 103.12799 95.295514) (width 0.29) (layer F.Cu) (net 23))
 (segment (start 101.14 75) (end 102.721968 76.581968) (width 0.29) (layer F.Cu) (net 23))
 (segment (start 105.3 99.6) (end 110.2 99.6) (width 0.29) (layer F.Cu) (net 23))
 (segment (start 103.371974 97.271974) (end 105.7 99.6) (width 0.29) (layer F.Cu) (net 23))
 (segment (start 105.605 102.165) (end 110.1 102.165) (width 0.29) (layer F.Cu) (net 22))
 (segment (start 100 80) (end 101.14 80) (width 0.29) (layer F.Cu) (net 22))
 (segment (start 102.279957 81.139957) (end 102.279957 92.629764) (width 0.29) (layer F.Cu) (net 22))
 (segment (start 102.68598 93.035786) (end 102.685981 95.478601) (width 0.29) (layer F.Cu) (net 22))
 (segment (start 102.929963 99.029963) (end 106.1 102.2) (width 0.29) (layer F.Cu) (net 22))
 (segment (start 102.685981 95.478601) (end 102.929963 95.722583) (width 0.29) (layer F.Cu) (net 22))
 (segment (start 102.279957 92.629764) (end 102.68598 93.035786) (width 0.29) (layer F.Cu) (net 22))
 (segment (start 101.14 80) (end 102.279957 81.139957) (width 0.29) (layer F.Cu) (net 22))
 (segment (start 102.929963 95.722583) (end 102.929963 99.029963) (width 0.29) (layer F.Cu) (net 22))
 (segment (start 101.837946 86.837946) (end 101.837946 92.81285) (width 0.29) (layer F.Cu) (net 21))
 (segment (start 102.243972 95.661688) (end 102.487952 95.905668) (width 0.29) (layer F.Cu) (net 21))
 (segment (start 100 85) (end 101.837946 86.837946) (width 0.29) (layer F.Cu) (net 21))
 (segment (start 105.5 104.7) (end 110.2 104.7) (width 0.29) (layer F.Cu) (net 21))
 (segment (start 101.837946 92.81285) (end 102.243971 93.218875) (width 0.29) (layer F.Cu) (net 21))
 (segment (start 102.243971 93.218875) (end 102.243972 95.661688) (width 0.29) (layer F.Cu) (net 21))
 (segment (start 102.487952 101.287952) (end 106 104.8) (width 0.29) (layer F.Cu) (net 21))
 (segment (start 102.487952 95.905668) (end 102.487952 101.287952) (width 0.29) (layer F.Cu) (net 21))
 (segment (start 105.5 107.3) (end 109.85 107.3) (width 0.29) (layer F.Cu) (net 20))
 (segment (start 102.045941 103.195941) (end 106.25 107.4) (width 0.29) (layer F.Cu) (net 20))
 (segment (start 100 91.6) (end 101.801962 93.401962) (width 0.29) (layer F.Cu) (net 20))
 (segment (start 101.801963 95.844775) (end 102.045941 96.088753) (width 0.29) (layer F.Cu) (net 20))
 (segment (start 100 90) (end 100 91.6) (width 0.29) (layer F.Cu) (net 20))
 (segment (start 101.801962 93.401962) (end 101.801963 95.844775) (width 0.29) (layer F.Cu) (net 20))
 (segment (start 102.045941 96.088753) (end 102.045941 103.195941) (width 0.29) (layer F.Cu) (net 20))
 (segment (start 101.226989 96.226989) (end 101.226989 103.126989) (width 0.152) (layer F.Cu) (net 19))
 (segment (start 102.8 104.7) (end 102.8 106.9) (width 0.152) (layer F.Cu) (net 19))
 (segment (start 100 95) (end 101.226989 96.226989) (width 0.152) (layer F.Cu) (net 19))
 (segment (start 101.226989 103.126989) (end 102.8 104.7) (width 0.152) (layer F.Cu) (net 19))
 (segment (start 105.3 109.8) (end 110.2 109.8) (width 0.152) (layer F.Cu) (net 19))
 (segment (start 102.8 106.9) (end 105.7 109.8) (width 0.152) (layer F.Cu) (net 19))
 (segment (start 101.9 108.4) (end 105.9 112.4) (width 0.152) (layer F.Cu) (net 18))
 (segment (start 101.9 104.4) (end 101.9 108.4) (width 0.152) (layer F.Cu) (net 18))
 (segment (start 100 102.5) (end 101.9 104.4) (width 0.152) (layer F.Cu) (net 18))
 (segment (start 100 100) (end 100 102.5) (width 0.152) (layer F.Cu) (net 18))
 (segment (start 105.6 112.3) (end 110.2 112.3) (width 0.152) (layer F.Cu) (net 18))
 (segment (start 105.4 114.9) (end 110.3 114.9) (width 0.152) (layer F.Cu) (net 17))
 (segment (start 101.4 110.6) (end 105.7 114.9) (width 0.152) (layer F.Cu) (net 17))
 (segment (start 100 105) (end 101.4 106.4) (width 0.152) (layer F.Cu) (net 17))
 (segment (start 101.4 106.4) (end 101.4 110.6) (width 0.152) (layer F.Cu) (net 17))
 (segment (start 100 110) (end 100 111.6) (width 1) (layer F.Cu) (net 16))
 (segment (start 100 111.6) (end 105.9 117.5) (width 1) (layer F.Cu) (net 16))
 (segment (start 105.87 117.405) (end 109.595 117.405) (width 1) (layer F.Cu) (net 16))
 (segment (start 100 115) (end 100.7 115) (width 1) (layer F.Cu) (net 15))
 (segment (start 100.7 115) (end 105.8 120.1) (width 1) (layer F.Cu) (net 15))
 (segment (start 105.87 119.945) (end 109.655 119.945) (width 1) (layer F.Cu) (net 15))
 (segment (start 109.655 119.945) (end 109.7 119.9) (width 1) (layer F.Cu) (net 15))
 (segment (start 100 120) (end 103.4 120) (width 1) (layer F.Cu) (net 14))
 (segment (start 103.4 120) (end 105.9 122.5) (width 1) (layer F.Cu) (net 14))
 (segment (start 105.87 122.485) (end 109.485 122.485) (width 1) (layer F.Cu) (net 14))
 (segment (start 109.485 122.485) (end 109.5 122.5) (width 1) (layer F.Cu) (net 14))
 (segment (start 100 125) (end 106 125) (width 0.152) (layer F.Cu) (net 13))
 (segment (start 105.7 125) (end 110.2 125) (width 0.152) (layer F.Cu) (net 13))
 (segment (start 100 130) (end 103.4 130) (width 1) (layer F.Cu) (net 12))
 (segment (start 103.4 130) (end 105.7 127.7) (width 1) (layer F.Cu) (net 12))
 (segment (start 105.87 127.565) (end 109.565 127.565) (width 1) (layer F.Cu) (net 12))
 (segment (start 109.565 127.565) (end 109.6 127.6) (width 1) (layer F.Cu) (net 12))
 (segment (start 100 135) (end 100.9 135) (width 1) (layer F.Cu) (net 11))
 (segment (start 100.9 135) (end 105.8 130.1) (width 1) (layer F.Cu) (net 11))
 (segment (start 105.87 130.105) (end 109.605 130.105) (width 1) (layer F.Cu) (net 11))
 (segment (start 109.605 130.105) (end 109.7 130.2) (width 1) (layer F.Cu) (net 11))
 (segment (start 101.502001 138.497999) (end 101.502001 136.897999) (width 1) (layer F.Cu) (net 10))
 (segment (start 100 140) (end 101.502001 138.497999) (width 1) (layer F.Cu) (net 10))
 (segment (start 101.502001 136.897999) (end 105.6 132.8) (width 1) (layer F.Cu) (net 10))
 (segment (start 105.87 132.645) (end 109.655 132.645) (width 1) (layer F.Cu) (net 10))
 (segment (start 109.655 132.645) (end 109.7 132.6) (width 1) (layer F.Cu) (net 10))
 (segment (start 100 145) (end 102.4 142.6) (width 0.152) (layer F.Cu) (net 9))
 (segment (start 102.4 138) (end 105.2 135.2) (width 0.152) (layer F.Cu) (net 9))
 (segment (start 102.4 142.6) (end 102.4 138) (width 0.152) (layer F.Cu) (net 9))
 (segment (start 105.87 135.185) (end 109.585 135.185) (width 0.152) (layer F.Cu) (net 9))
 (segment (start 109.585 135.185) (end 109.6 135.2) (width 0.152) (layer F.Cu) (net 9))
 (segment (start 100 150) (end 100 149.098) (width 0.152) (layer F.Cu) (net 8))
 (segment (start 103 146.098) (end 103 138.6) (width 0.152) (layer F.Cu) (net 8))
 (segment (start 103 138.6) (end 103.8 137.8) (width 0.152) (layer F.Cu) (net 8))
 (segment (start 100 149.098) (end 103 146.098) (width 0.152) (layer F.Cu) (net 8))
 (segment (start 103.8 137.8) (end 106 137.8) (width 0.152) (layer F.Cu) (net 8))
 (segment (start 106 137.8) (end 109.5 137.8) (width 0.152) (layer F.Cu) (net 8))
 (segment (start 109.5 137.8) (end 109.6 137.7) (width 0.152) (layer F.Cu) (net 8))
 (segment (start 103.30401 149.29599) (end 103.30401 141.39599) (width 0.152) (layer F.Cu) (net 7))
 (segment (start 103.30401 141.39599) (end 104.5 140.2) (width 0.152) (layer F.Cu) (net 7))
 (segment (start 100 155) (end 100 152.6) (width 0.152) (layer F.Cu) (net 7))
 (segment (start 100 152.6) (end 103.30401 149.29599) (width 0.152) (layer F.Cu) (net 7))
 (segment (start 104.5 140.2) (end 105.9 140.2) (width 0.152) (layer F.Cu) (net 7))
 (segment (start 105.9 140.2) (end 109.6 140.2) (width 0.152) (layer F.Cu) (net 7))
 (segment (start 101.3 158.7) (end 101.3 151.827516) (width 0.29) (layer F.Cu) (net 6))
 (segment (start 100 160) (end 101.3 158.7) (width 0.29) (layer F.Cu) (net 6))
 (segment (start 103.677021 149.450496) (end 103.677021 144.822979) (width 0.29) (layer F.Cu) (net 6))
 (segment (start 103.677021 144.822979) (end 105.7 142.8) (width 0.29) (layer F.Cu) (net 6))
 (segment (start 101.3 151.827516) (end 103.677021 149.450496) (width 0.29) (layer F.Cu) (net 6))
 (segment (start 105.4 142.8) (end 110.2 142.8) (width 0.29) (layer F.Cu) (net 6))
 (segment (start 105.6 145.3) (end 110.2 145.3) (width 0.29) (layer F.Cu) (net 5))
 (segment (start 101.837946 163.162054) (end 101.837946 151.914667) (width 0.29) (layer F.Cu) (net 5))
 (segment (start 104.5 147) (end 106 145.5) (width 0.29) (layer F.Cu) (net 5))
 (segment (start 101.837946 151.914667) (end 104.5 149.252613) (width 0.29) (layer F.Cu) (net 5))
 (segment (start 100 165) (end 101.837946 163.162054) (width 0.29) (layer F.Cu) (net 5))
 (segment (start 104.5 149.252613) (end 104.5 147) (width 0.29) (layer F.Cu) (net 5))
 (segment (start 106 147.9) (end 109.802562 147.9) (width 0.29) (layer F.Cu) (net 4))
 (segment (start 102.279957 152.317481) (end 106.597438 148) (width 0.29) (layer F.Cu) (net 4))
 (segment (start 100 170) (end 101.14 170) (width 0.29) (layer F.Cu) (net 4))
 (segment (start 102.279957 168.860043) (end 102.279957 152.317481) (width 0.29) (layer F.Cu) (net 4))
 (segment (start 101.14 170) (end 102.279957 168.860043) (width 0.29) (layer F.Cu) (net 4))
 (segment (start 100 175) (end 101.14 175) (width 0.29) (layer F.Cu) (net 3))
 (segment (start 101.14 175) (end 102.721968 173.418032) (width 0.29) (layer F.Cu) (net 3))
 (segment (start 102.721968 154.193923) (end 106.415891 150.5) (width 0.29) (layer F.Cu) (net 3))
 (segment (start 102.721968 173.418032) (end 102.721968 154.193923) (width 0.29) (layer F.Cu) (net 3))
 (segment (start 105.9 150.4) (end 110.084109 150.4) (width 0.29) (layer F.Cu) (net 3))
 (segment (start 110.2 153) (end 105.545 153) (width 0.35) (layer B.Cu) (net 2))
 (segment (start 105.7 153) (end 110.3 153) (width 0.35) (layer F.Cu) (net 2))
 (segment (start 103.6 155.23) (end 103.6 176.4) (width 0.35) (layer B.Cu) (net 2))
 (segment (start 105.865 152.965) (end 103.6 155.23) (width 0.35) (layer B.Cu) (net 2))
 (segment (start 103.5 155.4) (end 105.9 153) (width 0.35) (layer F.Cu) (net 2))
 (segment (start 103.6 176.4) (end 101.9 178.1) (width 0.35) (layer B.Cu) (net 2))
 (via (at 101.9 178.1) (size 0.6) (drill 0.3) (layers F.Cu B.Cu) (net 2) (status 1000000))
 (segment (start 103.5 176.5) (end 103.5 155.4) (width 0.35) (layer F.Cu) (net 2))
 (segment (start 101.9 178.1) (end 103.5 176.5) (width 0.35) (layer F.Cu) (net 2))
 (segment (start 100 180) (end 101.9 178.1) (width 1) (layer F.Cu) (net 2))
 (segment (start 100 185) (end 104.1 180.9) (width 0.152) (layer F.Cu) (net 1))
 (segment (start 104.1 180.9) (end 104.1 158.54219) (width 0.152) (layer F.Cu) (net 1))
 (segment (start 104.1 158.54219) (end 104.1 157.2) (width 0.152) (layer F.Cu) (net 1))
 (segment (start 104.1 157.2) (end 105.8 155.5) (width 0.152) (layer F.Cu) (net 1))
 (segment (start 105.8 155.5) (end 109.5 155.5) (width 0.152) (layer F.Cu) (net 1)))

